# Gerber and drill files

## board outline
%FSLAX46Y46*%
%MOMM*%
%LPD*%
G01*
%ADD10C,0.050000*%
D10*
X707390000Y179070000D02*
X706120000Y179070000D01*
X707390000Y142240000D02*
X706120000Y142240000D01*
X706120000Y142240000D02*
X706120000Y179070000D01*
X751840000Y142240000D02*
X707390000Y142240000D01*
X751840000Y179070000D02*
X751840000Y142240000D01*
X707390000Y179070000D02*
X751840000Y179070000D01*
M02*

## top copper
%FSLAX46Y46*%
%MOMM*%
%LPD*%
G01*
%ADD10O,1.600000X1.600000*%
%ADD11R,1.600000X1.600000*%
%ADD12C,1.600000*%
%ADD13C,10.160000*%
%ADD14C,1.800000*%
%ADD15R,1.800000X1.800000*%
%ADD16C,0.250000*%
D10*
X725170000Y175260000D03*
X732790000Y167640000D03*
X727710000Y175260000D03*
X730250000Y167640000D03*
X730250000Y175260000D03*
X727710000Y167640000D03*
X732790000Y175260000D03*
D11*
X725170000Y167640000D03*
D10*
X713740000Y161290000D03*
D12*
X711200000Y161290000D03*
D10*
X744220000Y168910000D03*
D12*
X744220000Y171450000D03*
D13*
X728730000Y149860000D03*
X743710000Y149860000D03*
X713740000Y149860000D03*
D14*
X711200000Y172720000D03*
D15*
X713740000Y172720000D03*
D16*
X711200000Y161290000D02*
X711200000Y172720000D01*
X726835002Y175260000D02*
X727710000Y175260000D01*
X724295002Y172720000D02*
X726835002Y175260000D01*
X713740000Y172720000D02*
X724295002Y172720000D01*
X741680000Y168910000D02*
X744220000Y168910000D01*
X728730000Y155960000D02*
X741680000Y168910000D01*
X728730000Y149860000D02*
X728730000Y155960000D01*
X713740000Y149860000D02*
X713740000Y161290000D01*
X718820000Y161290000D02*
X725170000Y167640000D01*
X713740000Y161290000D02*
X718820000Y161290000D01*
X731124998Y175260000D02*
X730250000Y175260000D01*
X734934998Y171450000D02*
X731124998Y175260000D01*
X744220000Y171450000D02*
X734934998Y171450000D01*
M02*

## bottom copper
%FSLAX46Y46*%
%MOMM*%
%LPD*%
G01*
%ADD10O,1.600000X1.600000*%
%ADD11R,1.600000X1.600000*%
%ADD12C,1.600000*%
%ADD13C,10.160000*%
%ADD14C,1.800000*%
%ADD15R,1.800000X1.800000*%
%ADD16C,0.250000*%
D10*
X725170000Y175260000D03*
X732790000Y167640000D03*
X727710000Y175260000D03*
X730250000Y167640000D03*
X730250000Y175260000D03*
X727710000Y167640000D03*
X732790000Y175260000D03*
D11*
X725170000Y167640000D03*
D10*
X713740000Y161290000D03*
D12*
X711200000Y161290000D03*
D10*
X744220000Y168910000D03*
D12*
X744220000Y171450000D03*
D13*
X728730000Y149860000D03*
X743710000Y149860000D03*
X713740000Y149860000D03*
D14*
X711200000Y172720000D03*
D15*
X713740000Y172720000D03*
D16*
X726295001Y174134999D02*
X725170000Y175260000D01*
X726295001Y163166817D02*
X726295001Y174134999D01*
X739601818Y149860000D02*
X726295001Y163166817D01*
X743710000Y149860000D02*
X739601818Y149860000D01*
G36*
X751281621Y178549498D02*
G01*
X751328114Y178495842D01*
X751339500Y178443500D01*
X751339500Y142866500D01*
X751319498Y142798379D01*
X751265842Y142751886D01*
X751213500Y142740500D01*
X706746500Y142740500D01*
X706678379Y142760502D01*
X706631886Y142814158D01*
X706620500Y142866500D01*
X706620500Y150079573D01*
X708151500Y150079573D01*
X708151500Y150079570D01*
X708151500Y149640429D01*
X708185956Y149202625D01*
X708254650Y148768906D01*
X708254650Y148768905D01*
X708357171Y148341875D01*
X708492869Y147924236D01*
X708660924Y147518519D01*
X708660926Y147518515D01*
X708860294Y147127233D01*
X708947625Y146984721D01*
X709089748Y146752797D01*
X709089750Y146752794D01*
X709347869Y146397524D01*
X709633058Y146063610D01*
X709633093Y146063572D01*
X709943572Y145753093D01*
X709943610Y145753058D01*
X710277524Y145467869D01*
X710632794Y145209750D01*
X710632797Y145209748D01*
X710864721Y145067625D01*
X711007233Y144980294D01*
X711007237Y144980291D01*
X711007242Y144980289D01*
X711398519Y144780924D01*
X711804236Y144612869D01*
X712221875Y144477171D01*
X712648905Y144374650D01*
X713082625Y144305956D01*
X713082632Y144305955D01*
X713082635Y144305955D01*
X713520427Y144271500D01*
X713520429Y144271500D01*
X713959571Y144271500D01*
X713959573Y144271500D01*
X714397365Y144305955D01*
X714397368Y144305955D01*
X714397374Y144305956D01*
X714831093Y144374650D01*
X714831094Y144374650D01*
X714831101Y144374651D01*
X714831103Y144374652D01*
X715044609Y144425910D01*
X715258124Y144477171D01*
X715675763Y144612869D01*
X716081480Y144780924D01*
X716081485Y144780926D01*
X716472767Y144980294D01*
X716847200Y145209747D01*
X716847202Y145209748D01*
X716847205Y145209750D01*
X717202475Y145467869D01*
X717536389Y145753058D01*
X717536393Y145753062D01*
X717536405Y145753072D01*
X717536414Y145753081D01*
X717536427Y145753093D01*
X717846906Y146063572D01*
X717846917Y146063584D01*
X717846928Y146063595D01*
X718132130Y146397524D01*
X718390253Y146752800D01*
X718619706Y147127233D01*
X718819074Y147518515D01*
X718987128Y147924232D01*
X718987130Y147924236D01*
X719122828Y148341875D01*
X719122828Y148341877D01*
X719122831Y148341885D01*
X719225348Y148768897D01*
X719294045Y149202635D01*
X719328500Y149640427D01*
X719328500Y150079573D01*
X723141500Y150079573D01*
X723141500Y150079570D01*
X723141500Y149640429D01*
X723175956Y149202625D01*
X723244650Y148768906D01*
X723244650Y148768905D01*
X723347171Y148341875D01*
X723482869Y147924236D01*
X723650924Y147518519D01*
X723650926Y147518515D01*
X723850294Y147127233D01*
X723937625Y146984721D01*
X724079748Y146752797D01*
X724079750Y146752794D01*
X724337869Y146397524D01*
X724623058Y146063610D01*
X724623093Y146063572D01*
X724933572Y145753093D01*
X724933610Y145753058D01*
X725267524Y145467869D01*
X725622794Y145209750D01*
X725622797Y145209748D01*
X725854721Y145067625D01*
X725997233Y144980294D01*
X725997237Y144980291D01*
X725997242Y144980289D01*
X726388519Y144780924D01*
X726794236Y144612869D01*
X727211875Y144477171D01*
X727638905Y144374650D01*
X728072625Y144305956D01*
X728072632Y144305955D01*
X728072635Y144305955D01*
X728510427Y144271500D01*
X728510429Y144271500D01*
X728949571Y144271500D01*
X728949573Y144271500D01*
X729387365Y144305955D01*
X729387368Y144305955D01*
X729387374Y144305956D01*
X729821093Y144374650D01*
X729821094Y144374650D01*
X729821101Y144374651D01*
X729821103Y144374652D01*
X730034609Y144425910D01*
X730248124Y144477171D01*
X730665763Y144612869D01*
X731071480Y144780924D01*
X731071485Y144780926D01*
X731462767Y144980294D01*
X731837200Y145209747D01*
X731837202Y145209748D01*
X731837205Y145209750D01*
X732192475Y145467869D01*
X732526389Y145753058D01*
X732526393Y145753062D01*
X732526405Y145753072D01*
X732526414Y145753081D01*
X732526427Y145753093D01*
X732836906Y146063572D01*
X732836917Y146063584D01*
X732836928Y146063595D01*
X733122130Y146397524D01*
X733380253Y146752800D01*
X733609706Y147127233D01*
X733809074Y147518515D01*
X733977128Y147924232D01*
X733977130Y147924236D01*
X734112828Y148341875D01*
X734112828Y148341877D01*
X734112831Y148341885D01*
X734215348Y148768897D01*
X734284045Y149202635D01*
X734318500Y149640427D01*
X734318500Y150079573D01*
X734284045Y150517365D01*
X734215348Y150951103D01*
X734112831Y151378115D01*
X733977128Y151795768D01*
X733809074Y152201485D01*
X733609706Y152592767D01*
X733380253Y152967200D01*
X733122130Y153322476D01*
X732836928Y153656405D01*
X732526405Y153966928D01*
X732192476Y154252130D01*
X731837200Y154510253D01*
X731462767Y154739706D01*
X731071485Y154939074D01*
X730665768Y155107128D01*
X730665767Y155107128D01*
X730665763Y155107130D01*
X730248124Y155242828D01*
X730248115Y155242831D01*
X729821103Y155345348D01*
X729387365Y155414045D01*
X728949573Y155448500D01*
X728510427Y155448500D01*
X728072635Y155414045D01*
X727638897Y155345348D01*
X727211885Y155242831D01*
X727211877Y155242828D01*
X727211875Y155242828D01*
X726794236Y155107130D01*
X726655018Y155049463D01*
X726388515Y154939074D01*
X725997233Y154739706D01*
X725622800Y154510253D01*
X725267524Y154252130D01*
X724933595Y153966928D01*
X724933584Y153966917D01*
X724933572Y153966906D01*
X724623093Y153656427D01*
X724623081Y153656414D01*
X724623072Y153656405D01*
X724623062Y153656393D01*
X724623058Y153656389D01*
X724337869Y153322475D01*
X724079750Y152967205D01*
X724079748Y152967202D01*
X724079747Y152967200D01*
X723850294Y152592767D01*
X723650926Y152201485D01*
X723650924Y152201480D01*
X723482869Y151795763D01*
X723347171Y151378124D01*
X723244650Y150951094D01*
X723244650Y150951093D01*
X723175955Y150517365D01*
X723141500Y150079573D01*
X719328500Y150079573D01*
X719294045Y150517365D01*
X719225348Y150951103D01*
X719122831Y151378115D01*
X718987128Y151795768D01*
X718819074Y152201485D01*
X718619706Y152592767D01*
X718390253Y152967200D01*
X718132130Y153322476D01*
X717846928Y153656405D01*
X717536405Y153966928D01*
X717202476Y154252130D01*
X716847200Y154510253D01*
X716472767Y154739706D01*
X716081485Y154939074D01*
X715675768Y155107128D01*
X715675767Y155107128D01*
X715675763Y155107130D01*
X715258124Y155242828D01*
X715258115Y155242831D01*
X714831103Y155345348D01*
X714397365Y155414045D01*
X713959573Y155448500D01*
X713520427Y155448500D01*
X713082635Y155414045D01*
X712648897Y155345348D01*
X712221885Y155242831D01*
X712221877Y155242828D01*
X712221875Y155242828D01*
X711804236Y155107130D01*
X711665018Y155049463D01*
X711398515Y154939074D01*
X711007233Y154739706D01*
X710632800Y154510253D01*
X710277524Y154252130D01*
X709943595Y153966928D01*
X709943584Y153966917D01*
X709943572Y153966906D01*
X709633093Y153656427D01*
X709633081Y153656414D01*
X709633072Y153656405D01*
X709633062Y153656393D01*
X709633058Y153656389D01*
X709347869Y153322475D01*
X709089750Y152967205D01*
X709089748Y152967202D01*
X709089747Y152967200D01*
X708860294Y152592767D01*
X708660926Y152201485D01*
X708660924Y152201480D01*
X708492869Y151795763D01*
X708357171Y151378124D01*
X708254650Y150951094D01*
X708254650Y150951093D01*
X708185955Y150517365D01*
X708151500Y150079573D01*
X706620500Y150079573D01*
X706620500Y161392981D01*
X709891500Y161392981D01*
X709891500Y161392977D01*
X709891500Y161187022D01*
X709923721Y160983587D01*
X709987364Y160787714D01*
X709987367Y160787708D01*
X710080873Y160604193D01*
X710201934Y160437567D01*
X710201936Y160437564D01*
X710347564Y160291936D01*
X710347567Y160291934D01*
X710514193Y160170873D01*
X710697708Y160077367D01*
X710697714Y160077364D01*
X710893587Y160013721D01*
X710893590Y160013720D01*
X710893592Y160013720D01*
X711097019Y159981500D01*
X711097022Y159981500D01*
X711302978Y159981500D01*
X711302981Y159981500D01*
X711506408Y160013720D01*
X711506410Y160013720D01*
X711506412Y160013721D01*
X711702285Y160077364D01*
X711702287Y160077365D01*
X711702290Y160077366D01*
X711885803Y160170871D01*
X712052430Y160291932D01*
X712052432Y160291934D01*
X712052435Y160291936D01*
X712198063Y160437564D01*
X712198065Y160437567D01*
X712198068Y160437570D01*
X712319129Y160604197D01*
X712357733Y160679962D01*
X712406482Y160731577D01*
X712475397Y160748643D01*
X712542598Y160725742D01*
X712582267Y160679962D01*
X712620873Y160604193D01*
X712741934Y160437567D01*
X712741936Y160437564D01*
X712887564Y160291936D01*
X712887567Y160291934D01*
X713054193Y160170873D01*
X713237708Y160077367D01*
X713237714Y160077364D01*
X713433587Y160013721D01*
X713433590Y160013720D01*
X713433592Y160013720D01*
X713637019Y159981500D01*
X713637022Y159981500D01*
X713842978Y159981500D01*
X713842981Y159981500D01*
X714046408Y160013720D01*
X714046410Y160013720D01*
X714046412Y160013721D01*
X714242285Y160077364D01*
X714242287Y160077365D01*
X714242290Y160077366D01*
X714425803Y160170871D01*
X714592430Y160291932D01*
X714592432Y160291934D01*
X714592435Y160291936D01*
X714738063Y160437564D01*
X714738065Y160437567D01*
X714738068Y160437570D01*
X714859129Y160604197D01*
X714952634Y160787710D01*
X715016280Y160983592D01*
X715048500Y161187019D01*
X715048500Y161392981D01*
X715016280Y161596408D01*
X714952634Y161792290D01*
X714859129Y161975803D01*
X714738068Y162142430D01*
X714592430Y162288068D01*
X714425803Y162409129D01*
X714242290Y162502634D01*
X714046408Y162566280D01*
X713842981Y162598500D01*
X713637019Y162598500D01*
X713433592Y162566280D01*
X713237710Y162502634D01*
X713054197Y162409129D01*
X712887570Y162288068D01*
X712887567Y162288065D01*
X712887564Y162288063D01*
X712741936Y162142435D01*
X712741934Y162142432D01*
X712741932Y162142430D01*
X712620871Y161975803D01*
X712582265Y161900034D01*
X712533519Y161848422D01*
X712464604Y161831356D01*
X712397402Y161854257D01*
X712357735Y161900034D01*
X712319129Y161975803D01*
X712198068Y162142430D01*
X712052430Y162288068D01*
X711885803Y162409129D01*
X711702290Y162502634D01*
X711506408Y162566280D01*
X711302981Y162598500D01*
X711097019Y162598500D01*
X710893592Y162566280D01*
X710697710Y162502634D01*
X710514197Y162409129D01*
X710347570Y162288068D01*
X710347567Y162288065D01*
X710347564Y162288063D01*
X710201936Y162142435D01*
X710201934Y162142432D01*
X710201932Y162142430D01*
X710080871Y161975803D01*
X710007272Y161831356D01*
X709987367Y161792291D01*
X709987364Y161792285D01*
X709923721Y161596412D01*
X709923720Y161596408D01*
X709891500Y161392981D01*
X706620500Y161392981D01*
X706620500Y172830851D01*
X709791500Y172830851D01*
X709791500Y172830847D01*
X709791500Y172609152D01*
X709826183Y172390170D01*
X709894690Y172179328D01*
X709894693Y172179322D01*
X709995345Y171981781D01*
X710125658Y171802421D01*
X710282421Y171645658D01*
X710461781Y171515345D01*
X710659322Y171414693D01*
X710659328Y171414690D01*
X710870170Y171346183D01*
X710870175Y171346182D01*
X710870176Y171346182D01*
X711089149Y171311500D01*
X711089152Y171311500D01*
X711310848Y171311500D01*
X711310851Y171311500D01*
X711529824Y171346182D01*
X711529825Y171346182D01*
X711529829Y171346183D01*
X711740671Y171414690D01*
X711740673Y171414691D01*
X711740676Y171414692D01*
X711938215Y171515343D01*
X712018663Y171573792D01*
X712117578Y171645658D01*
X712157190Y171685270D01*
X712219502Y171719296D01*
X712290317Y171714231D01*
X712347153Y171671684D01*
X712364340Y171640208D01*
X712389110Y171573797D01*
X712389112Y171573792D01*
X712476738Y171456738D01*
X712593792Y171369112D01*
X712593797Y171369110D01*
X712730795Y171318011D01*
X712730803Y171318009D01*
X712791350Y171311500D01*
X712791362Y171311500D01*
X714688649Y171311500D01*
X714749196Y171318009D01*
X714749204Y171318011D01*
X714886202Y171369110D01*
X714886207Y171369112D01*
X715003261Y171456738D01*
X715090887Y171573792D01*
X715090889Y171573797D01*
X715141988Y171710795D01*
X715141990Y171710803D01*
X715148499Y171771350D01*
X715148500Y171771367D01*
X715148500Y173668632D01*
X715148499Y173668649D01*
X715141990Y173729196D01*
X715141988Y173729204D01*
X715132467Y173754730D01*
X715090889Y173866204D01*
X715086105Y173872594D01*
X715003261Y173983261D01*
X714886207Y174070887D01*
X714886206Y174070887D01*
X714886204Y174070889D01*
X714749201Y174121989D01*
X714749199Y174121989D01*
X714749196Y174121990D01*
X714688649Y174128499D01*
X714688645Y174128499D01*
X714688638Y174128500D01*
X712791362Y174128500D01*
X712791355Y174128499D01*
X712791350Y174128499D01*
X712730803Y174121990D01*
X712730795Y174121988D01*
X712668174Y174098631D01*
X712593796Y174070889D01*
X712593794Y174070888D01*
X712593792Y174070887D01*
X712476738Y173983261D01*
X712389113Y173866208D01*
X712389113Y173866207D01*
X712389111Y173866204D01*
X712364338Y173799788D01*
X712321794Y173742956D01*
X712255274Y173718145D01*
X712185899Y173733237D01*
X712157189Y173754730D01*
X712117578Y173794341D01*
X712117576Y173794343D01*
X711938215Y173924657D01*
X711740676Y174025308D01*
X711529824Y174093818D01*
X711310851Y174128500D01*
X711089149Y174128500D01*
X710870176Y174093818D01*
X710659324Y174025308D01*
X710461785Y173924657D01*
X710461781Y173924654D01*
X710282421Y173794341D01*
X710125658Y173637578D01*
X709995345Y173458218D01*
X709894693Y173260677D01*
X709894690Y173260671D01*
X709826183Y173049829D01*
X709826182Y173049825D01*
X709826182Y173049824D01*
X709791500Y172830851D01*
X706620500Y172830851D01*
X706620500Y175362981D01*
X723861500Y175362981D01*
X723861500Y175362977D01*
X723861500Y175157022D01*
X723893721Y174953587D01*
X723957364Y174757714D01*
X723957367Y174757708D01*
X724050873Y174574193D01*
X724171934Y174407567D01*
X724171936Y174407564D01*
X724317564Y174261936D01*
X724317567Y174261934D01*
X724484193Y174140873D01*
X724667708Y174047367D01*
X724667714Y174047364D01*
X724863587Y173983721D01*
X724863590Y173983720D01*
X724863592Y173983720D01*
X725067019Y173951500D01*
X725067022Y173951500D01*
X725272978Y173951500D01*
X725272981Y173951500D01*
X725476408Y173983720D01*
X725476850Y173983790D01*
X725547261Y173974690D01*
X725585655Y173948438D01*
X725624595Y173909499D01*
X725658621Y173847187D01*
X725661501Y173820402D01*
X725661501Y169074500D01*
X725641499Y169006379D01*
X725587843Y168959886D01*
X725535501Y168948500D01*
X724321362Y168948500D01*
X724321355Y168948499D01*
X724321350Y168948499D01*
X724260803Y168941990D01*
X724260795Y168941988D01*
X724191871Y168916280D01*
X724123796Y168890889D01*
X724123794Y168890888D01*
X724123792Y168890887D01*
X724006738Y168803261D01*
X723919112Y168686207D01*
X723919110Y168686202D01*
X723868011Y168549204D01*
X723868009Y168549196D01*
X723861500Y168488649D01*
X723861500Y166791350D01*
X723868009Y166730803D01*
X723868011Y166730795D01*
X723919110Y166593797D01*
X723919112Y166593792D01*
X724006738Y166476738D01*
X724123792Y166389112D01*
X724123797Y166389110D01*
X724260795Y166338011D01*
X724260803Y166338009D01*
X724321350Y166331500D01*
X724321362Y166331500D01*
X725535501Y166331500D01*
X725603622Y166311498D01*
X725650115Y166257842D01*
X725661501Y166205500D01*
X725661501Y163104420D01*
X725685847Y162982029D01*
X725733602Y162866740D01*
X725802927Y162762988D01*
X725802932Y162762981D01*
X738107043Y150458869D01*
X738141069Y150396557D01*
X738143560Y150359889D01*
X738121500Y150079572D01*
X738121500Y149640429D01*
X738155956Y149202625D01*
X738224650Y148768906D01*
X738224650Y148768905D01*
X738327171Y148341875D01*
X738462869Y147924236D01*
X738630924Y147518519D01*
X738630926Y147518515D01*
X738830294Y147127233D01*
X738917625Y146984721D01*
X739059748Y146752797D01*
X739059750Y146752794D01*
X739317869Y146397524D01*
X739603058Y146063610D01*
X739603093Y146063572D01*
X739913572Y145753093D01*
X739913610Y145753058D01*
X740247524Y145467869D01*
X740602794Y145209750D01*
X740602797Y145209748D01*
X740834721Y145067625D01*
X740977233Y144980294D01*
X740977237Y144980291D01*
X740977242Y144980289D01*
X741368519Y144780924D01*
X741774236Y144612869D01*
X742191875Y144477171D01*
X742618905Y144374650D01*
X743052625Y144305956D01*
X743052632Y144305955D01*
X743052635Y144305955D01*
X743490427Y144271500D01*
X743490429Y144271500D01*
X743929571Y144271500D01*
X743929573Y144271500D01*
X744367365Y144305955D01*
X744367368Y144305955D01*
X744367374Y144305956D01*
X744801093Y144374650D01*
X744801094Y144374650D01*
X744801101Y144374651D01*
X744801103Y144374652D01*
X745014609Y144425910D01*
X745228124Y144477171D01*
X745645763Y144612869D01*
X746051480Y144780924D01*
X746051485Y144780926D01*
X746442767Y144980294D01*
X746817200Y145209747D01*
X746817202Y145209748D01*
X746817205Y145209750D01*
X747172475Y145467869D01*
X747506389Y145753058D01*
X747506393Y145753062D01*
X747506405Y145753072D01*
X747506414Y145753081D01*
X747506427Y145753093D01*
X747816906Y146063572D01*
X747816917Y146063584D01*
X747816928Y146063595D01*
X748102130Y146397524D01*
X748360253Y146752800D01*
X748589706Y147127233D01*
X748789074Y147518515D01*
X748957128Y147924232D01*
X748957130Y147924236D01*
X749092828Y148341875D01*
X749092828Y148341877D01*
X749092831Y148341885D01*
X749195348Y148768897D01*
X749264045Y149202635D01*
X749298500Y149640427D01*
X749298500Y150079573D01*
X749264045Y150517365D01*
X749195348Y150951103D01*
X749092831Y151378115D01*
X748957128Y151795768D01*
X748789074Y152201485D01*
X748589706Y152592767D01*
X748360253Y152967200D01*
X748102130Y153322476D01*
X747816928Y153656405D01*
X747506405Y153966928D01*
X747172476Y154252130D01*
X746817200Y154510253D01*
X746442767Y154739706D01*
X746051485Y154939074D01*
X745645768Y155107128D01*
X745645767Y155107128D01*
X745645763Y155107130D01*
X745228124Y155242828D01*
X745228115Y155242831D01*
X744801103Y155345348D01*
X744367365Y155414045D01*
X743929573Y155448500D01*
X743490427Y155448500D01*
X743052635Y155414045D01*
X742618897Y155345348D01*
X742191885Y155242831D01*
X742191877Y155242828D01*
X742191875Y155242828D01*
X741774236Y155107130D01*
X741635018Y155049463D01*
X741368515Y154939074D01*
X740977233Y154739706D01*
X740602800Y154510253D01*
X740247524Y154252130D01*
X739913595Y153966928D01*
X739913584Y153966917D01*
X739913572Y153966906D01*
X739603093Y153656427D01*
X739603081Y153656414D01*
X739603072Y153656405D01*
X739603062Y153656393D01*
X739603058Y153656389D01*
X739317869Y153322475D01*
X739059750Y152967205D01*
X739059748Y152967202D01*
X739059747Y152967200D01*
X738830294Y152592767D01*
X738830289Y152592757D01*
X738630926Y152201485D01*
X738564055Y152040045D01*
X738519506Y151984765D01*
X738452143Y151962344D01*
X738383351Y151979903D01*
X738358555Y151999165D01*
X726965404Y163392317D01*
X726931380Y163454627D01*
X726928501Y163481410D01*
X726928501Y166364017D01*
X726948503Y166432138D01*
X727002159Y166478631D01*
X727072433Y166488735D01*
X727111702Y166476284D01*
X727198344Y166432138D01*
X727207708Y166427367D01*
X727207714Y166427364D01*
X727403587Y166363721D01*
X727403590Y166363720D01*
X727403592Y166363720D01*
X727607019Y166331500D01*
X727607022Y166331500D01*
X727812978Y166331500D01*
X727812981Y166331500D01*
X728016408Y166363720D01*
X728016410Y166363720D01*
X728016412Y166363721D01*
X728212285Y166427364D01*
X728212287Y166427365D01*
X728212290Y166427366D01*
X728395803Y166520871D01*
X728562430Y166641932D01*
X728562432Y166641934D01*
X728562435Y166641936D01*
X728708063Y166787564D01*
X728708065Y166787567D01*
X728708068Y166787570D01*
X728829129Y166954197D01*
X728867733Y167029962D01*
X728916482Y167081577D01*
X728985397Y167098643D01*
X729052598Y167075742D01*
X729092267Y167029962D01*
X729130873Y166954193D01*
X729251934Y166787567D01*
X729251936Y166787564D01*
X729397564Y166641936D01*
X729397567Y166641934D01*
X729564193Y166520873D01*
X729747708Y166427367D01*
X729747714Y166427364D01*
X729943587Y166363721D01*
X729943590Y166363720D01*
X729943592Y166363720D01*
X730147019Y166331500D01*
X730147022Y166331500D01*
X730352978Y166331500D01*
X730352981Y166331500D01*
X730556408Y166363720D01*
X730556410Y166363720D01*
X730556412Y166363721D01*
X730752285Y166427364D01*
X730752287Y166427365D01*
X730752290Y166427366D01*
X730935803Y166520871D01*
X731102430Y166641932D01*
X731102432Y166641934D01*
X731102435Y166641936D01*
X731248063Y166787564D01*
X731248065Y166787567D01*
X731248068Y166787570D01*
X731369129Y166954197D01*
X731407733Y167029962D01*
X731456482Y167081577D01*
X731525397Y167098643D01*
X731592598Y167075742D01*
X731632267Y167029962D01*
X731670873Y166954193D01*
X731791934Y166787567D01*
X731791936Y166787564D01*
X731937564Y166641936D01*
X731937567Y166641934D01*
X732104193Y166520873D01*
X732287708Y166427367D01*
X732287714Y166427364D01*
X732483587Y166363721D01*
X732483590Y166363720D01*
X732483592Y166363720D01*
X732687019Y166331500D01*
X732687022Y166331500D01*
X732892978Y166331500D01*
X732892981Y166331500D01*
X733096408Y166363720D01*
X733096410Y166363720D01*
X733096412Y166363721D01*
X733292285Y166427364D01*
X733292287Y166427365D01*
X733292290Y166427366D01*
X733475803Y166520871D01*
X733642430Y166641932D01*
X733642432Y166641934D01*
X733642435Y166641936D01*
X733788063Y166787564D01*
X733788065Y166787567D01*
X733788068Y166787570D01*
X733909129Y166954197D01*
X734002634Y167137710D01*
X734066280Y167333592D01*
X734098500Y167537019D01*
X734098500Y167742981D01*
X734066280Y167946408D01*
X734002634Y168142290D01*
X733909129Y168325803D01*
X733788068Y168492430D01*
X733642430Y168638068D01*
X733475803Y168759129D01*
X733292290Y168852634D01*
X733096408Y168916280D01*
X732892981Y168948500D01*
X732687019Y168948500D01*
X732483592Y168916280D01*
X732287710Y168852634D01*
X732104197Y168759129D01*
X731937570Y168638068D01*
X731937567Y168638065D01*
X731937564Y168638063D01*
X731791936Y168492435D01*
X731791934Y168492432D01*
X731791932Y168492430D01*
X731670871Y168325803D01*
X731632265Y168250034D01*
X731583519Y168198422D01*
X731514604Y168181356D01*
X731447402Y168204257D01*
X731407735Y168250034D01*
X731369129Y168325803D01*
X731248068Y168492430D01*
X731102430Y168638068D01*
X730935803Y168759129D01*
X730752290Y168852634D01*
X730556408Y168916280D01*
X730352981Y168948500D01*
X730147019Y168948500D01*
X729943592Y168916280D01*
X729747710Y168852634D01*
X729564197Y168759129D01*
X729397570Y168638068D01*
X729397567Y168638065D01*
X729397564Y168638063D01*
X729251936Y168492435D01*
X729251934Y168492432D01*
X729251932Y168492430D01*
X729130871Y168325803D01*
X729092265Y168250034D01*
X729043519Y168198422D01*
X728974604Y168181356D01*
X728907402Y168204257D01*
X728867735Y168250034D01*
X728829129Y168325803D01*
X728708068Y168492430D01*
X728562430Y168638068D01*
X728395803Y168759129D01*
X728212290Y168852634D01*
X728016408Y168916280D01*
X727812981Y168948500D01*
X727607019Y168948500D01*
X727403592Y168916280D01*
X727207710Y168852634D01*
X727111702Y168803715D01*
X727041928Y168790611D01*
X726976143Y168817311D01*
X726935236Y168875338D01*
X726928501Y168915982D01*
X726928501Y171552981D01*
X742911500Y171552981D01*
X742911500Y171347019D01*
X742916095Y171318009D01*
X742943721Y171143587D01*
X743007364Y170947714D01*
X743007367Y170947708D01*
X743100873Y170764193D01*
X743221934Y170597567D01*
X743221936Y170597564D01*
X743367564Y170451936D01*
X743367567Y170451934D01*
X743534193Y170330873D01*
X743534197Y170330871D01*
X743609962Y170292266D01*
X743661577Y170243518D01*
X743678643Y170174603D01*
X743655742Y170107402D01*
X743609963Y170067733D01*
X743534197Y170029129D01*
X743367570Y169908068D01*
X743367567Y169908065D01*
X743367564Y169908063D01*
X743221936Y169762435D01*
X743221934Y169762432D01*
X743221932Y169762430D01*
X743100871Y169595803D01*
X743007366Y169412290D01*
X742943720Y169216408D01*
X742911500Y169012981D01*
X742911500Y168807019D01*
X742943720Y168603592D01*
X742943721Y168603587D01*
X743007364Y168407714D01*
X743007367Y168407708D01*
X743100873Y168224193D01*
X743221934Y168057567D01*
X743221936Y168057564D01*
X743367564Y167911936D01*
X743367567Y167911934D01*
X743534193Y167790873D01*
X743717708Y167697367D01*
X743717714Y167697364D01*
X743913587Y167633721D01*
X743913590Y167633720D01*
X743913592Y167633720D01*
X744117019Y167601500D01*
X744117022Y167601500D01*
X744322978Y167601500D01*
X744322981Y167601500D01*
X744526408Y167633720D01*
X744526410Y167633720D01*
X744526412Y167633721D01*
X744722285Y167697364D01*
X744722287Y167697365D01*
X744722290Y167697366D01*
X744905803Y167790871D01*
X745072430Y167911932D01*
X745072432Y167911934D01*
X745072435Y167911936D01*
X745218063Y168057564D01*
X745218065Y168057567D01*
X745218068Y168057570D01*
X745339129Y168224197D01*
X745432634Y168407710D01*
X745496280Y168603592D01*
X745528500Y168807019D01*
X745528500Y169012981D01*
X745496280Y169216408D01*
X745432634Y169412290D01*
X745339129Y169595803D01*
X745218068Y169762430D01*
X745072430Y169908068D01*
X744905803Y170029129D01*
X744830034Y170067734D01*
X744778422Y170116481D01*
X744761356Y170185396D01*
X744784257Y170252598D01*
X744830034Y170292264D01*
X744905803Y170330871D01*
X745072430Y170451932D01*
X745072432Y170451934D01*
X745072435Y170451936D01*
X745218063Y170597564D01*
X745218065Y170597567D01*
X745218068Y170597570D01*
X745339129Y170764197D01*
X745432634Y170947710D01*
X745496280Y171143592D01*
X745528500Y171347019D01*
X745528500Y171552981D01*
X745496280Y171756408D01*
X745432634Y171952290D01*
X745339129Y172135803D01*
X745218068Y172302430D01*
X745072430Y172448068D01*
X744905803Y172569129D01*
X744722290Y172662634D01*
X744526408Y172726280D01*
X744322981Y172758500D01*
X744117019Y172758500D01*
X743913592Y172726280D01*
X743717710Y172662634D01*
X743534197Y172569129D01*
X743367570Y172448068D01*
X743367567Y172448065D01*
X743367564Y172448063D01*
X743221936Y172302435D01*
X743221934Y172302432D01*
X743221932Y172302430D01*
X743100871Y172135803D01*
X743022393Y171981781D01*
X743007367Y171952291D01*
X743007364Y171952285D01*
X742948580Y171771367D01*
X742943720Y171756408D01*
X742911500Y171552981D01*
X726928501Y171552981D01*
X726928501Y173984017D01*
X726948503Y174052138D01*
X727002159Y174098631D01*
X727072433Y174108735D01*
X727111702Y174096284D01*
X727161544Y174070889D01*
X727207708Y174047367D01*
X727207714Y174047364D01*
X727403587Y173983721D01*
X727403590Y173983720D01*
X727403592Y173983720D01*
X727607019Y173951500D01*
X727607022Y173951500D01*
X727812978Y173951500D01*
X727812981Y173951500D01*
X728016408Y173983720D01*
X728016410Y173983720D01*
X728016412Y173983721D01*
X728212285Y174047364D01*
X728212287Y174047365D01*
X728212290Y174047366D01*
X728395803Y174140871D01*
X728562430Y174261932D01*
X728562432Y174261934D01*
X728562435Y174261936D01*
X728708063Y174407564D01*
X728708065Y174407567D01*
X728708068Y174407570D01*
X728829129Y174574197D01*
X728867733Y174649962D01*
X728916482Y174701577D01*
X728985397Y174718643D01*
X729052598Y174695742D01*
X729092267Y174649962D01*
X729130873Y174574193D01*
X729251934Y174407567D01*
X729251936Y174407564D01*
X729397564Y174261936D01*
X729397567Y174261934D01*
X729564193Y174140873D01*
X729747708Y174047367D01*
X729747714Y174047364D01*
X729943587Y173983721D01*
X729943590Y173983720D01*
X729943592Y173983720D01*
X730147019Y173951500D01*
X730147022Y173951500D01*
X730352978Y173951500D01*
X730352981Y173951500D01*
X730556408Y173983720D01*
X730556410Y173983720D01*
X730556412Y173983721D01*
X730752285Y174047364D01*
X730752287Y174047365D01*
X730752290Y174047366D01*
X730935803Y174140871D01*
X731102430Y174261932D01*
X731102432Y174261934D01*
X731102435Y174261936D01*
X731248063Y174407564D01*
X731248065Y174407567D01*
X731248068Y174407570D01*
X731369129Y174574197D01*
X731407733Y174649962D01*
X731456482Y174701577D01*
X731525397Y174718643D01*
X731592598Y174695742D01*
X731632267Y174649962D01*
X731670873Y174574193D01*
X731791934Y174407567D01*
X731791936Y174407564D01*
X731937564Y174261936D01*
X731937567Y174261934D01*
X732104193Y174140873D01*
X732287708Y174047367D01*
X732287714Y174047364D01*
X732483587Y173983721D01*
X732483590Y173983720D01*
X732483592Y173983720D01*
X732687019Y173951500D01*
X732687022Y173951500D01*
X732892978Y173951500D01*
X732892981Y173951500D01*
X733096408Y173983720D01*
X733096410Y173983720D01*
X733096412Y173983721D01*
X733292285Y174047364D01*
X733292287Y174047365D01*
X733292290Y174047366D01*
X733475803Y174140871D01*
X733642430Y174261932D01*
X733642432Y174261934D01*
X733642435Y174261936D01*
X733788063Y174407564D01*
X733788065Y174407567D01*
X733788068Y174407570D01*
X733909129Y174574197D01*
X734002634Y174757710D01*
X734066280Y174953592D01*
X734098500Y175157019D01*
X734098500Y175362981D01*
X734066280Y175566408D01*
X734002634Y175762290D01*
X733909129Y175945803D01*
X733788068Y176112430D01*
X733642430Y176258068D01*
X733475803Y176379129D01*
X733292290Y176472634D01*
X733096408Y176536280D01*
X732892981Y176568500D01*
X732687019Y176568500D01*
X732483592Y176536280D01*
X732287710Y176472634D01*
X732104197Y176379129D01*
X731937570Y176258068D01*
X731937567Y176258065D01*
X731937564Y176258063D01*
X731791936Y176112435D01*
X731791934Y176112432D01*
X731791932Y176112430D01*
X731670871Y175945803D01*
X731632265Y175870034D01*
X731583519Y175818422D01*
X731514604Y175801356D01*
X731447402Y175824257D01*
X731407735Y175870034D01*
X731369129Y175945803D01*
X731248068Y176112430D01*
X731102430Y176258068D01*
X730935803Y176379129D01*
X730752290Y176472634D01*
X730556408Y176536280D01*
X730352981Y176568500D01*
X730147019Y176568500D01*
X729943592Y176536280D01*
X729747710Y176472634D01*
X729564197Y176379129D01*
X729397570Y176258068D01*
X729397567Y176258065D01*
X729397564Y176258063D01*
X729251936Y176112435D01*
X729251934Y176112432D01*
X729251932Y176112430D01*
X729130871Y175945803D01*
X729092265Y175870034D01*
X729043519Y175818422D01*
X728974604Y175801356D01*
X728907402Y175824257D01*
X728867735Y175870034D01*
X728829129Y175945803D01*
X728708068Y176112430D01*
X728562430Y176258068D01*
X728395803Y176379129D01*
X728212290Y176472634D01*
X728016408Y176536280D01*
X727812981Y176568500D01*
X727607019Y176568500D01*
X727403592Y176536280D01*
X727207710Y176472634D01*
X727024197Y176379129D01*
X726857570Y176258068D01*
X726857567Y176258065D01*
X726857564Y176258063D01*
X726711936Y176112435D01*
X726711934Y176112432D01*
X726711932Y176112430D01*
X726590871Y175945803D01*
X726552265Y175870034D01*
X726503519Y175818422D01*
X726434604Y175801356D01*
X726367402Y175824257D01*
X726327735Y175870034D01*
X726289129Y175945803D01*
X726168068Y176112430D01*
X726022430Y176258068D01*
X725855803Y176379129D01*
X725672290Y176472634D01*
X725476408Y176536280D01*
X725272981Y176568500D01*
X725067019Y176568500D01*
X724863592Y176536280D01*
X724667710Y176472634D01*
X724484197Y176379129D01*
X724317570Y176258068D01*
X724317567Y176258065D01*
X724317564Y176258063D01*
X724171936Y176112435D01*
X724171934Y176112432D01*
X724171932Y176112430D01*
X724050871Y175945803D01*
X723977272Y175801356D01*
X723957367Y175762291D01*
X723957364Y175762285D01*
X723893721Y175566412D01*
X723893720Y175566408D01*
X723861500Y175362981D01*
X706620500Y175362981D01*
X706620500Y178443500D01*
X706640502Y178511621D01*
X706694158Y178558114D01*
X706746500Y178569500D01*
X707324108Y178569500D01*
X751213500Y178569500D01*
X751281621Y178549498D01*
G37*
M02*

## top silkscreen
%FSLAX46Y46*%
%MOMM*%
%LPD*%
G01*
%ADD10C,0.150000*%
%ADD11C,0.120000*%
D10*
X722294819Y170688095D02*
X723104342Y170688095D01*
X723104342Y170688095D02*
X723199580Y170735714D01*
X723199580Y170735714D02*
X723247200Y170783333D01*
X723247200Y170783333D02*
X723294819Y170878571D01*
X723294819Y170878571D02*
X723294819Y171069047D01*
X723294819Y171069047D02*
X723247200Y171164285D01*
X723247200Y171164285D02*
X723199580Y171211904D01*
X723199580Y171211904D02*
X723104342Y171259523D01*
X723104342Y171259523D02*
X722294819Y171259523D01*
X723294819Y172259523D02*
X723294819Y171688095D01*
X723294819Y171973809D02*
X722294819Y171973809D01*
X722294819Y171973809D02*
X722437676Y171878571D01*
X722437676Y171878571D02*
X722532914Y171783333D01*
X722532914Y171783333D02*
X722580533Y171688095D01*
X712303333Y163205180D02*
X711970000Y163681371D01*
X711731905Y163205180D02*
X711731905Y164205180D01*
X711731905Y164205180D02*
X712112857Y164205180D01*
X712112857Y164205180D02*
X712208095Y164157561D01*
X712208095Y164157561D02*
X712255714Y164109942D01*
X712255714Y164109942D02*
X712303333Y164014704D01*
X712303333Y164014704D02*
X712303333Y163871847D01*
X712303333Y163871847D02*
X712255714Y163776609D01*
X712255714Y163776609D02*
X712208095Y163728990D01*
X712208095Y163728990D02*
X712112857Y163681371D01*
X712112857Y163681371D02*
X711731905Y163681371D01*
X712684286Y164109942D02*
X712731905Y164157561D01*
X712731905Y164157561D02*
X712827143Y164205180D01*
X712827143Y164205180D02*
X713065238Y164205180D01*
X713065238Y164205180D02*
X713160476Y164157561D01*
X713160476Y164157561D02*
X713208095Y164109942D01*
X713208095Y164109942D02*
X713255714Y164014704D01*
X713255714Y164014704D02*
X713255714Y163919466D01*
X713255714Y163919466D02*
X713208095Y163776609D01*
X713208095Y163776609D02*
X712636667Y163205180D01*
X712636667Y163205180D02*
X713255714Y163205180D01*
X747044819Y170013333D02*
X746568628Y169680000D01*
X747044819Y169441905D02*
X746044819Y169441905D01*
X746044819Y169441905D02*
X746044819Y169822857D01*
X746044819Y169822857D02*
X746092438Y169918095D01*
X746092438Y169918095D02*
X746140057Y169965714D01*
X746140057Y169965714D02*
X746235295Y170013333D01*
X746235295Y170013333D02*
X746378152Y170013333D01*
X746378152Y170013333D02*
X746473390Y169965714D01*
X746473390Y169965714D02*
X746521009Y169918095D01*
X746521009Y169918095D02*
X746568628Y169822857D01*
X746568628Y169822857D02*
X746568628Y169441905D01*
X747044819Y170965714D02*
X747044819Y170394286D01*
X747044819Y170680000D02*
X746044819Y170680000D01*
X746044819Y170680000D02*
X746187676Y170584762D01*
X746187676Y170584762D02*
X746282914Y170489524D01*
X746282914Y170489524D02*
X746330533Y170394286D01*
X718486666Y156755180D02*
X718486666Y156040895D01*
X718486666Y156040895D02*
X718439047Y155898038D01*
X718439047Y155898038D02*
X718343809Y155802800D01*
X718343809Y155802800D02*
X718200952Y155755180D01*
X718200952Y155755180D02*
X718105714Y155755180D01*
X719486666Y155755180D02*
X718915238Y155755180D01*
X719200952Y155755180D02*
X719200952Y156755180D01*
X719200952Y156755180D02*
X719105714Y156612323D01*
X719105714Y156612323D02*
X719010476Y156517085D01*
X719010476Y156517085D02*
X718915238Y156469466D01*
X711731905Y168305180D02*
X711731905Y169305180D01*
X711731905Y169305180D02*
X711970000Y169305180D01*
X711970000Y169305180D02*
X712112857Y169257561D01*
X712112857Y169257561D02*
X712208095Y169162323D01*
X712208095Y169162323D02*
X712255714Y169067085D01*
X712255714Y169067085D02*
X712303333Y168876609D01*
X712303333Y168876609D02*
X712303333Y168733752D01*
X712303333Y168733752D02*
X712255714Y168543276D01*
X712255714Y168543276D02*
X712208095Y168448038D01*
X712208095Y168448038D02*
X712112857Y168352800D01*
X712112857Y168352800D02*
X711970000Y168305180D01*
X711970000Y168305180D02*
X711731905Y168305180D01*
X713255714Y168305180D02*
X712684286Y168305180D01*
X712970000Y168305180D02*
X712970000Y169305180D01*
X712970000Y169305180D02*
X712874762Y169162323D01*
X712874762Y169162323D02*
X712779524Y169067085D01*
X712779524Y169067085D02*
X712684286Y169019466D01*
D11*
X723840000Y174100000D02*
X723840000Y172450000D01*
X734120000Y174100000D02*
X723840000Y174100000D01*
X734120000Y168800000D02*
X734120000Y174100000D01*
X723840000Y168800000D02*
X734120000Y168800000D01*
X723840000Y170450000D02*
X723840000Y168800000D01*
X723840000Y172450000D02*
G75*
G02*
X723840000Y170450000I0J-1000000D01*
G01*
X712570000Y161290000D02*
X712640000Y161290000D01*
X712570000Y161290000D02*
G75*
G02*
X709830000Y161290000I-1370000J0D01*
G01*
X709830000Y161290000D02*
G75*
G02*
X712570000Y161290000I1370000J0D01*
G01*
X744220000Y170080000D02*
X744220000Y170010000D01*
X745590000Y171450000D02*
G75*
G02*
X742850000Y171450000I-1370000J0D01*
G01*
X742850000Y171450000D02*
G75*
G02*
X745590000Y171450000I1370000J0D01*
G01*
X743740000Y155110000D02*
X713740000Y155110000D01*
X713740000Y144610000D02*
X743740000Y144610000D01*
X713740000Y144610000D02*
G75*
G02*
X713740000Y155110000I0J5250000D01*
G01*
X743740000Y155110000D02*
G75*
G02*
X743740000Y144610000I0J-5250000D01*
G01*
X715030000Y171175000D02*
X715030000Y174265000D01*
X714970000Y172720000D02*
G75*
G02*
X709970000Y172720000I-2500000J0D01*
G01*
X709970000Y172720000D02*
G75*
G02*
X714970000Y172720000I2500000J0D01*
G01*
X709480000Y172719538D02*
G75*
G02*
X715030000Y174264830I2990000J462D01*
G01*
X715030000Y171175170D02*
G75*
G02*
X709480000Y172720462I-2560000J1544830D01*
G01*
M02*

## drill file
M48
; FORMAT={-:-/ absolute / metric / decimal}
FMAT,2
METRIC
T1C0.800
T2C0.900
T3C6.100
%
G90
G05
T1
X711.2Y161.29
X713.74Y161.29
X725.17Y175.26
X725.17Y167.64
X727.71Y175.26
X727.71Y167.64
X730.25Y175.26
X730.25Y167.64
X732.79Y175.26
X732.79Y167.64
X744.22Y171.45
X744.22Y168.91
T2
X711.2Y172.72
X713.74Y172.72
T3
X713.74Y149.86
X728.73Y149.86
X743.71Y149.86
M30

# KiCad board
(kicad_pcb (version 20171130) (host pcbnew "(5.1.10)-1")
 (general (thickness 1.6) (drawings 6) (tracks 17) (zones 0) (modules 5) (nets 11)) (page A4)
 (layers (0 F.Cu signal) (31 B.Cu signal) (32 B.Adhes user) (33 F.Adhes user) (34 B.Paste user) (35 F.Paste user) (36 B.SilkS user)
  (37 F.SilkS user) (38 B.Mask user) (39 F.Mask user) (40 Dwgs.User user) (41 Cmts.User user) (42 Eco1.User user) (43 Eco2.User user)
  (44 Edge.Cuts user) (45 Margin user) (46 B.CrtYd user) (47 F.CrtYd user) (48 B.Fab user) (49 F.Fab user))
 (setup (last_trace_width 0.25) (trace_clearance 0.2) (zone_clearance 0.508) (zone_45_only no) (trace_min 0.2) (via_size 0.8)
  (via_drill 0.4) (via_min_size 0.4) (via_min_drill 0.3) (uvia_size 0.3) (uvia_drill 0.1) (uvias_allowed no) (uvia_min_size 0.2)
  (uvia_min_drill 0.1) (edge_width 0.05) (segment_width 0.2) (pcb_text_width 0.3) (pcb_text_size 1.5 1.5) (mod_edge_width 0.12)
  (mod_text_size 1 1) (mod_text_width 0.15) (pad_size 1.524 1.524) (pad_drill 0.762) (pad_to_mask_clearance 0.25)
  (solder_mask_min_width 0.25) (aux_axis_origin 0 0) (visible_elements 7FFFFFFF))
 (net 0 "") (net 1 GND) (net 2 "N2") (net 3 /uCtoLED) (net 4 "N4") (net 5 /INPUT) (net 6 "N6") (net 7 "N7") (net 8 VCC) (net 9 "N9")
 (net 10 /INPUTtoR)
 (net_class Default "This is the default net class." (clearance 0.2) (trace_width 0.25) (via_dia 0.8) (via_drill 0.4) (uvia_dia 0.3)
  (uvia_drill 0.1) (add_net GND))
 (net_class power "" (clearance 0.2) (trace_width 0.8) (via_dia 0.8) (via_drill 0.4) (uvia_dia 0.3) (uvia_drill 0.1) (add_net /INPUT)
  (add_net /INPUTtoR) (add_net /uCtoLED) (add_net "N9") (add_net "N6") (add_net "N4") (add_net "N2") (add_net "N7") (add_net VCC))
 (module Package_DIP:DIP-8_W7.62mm (layer F.Cu) (at 725.17 -167.64 90)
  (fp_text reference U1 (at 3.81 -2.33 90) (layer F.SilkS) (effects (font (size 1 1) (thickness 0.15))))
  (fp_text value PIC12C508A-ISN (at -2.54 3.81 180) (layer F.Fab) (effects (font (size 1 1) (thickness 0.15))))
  (fp_line (start 6.46 -1.33) (end 4.81 -1.33) (layer F.SilkS) (width 0.12))
  (fp_line (start 6.46 8.95) (end 6.46 -1.33) (layer F.SilkS) (width 0.12))
  (fp_line (start 1.16 8.95) (end 6.46 8.95) (layer F.SilkS) (width 0.12))
  (fp_line (start 1.16 -1.33) (end 1.16 8.95) (layer F.SilkS) (width 0.12))
  (fp_line (start 2.81 -1.33) (end 1.16 -1.33) (layer F.SilkS) (width 0.12))
  (fp_arc (start 3.81 -1.33) (end 2.81 -1.33) (angle -180) (layer F.SilkS) (width 0.12))
  (pad 8 thru_hole oval (at 7.62 0 90) (size 1.6 1.6) (drill 0.8) (layers *.Cu *.Mask) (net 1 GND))
  (pad 4 thru_hole oval (at 0 7.62 90) (size 1.6 1.6) (drill 0.8) (layers *.Cu *.Mask) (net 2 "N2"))
  (pad 7 thru_hole oval (at 7.62 2.54 90) (size 1.6 1.6) (drill 0.8) (layers *.Cu *.Mask) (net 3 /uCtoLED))
  (pad 3 thru_hole oval (at 0 5.08 90) (size 1.6 1.6) (drill 0.8) (layers *.Cu *.Mask) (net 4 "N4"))
  (pad 6 thru_hole oval (at 7.62 5.08 90) (size 1.6 1.6) (drill 0.8) (layers *.Cu *.Mask) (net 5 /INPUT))
  (pad 2 thru_hole oval (at 0 2.54 90) (size 1.6 1.6) (drill 0.8) (layers *.Cu *.Mask) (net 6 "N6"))
  (pad 5 thru_hole oval (at 7.62 7.62 90) (size 1.6 1.6) (drill 0.8) (layers *.Cu *.Mask) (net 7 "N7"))
  (pad 1 thru_hole rect (at 0 0 90) (size 1.6 1.6) (drill 0.8) (layers *.Cu *.Mask) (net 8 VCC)))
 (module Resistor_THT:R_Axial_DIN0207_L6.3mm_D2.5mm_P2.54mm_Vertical (layer F.Cu) (at 711.2 -161.29)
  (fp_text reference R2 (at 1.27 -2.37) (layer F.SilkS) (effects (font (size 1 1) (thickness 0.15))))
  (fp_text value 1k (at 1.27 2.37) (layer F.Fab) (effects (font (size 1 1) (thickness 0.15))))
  (fp_line (start 1.37 0) (end 1.44 0) (layer F.SilkS) (width 0.12))
  (fp_circle (center 0 0) (end 1.37 0) (layer F.SilkS) (width 0.12))
  (pad 2 thru_hole oval (at 2.54 0) (size 1.6 1.6) (drill 0.8) (layers *.Cu *.Mask) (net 8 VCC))
  (pad 1 thru_hole circle (at 0 0) (size 1.6 1.6) (drill 0.8) (layers *.Cu *.Mask) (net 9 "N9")))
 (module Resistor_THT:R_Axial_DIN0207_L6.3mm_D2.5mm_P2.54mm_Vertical (layer F.Cu) (at 744.22 -171.45 270)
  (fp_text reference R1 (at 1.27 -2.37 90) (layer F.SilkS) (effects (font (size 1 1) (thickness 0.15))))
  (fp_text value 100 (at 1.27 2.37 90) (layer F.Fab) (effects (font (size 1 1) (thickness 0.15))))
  (fp_line (start 1.37 0) (end 1.44 0) (layer F.SilkS) (width 0.12))
  (fp_circle (center 0 0) (end 1.37 0) (layer F.SilkS) (width 0.12))
  (pad 2 thru_hole oval (at 2.54 0 270) (size 1.6 1.6) (drill 0.8) (layers *.Cu *.Mask) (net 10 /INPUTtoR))
  (pad 1 thru_hole circle (at 0 0 270) (size 1.6 1.6) (drill 0.8) (layers *.Cu *.Mask) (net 5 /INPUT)))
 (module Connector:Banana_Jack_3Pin (layer F.Cu) (at 713.74 -149.86)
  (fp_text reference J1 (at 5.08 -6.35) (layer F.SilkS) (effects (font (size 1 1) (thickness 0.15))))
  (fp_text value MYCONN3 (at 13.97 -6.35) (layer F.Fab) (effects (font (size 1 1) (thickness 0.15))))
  (fp_line (start 30 -5.25) (end 0 -5.25) (layer F.SilkS) (width 0.12))
  (fp_line (start 0 5.25) (end 30 5.25) (layer F.SilkS) (width 0.12))
  (fp_arc (start 0 0) (end 0 5.25) (angle 180) (layer F.SilkS) (width 0.12))
  (fp_arc (start 30 0) (end 30 -5.25) (angle 180) (layer F.SilkS) (width 0.12))
  (pad 2 thru_hole circle (at 14.99 0) (size 10.16 10.16) (drill 6.1) (layers *.Cu *.Mask) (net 10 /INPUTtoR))
  (pad 3 thru_hole circle (at 29.97 0) (size 10.16 10.16) (drill 6.1) (layers *.Cu *.Mask) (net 1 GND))
  (pad 1 thru_hole circle (at 0 0) (size 10.16 10.16) (drill 6.1) (layers *.Cu *.Mask) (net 8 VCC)))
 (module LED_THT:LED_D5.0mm (layer F.Cu) (at 713.74 -172.72 180)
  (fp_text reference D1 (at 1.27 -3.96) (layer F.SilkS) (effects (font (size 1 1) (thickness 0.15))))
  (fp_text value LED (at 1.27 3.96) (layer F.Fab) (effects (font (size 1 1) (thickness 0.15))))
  (fp_line (start -1.29 -1.545) (end -1.29 1.545) (layer F.SilkS) (width 0.12))
  (fp_circle (center 1.27 0) (end 3.77 0) (layer F.SilkS) (width 0.12))
  (fp_arc (start 1.27 0) (end -1.29 1.54483) (angle -148.9) (layer F.SilkS) (width 0.12))
  (fp_arc (start 1.27 0) (end -1.29 -1.54483) (angle 148.9) (layer F.SilkS) (width 0.12))
  (pad 2 thru_hole circle (at 2.54 0 180) (size 1.8 1.8) (drill 0.9) (layers *.Cu *.Mask) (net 9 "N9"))
  (pad 1 thru_hole rect (at 0 0 180) (size 1.8 1.8) (drill 0.9) (layers *.Cu *.Mask) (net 3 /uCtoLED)))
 (gr_line (start 707.39 -179.07) (end 706.12 -179.07) (layer Edge.Cuts) (width 0.05))
 (gr_line (start 707.39 -142.24) (end 706.12 -142.24) (layer Edge.Cuts) (width 0.05))
 (gr_line (start 706.12 -142.24) (end 706.12 -179.07) (layer Edge.Cuts) (width 0.05))
 (gr_line (start 751.84 -142.24) (end 707.39 -142.24) (layer Edge.Cuts) (width 0.05))
 (gr_line (start 751.84 -179.07) (end 751.84 -142.24) (layer Edge.Cuts) (width 0.05))
 (gr_line (start 707.39 -179.07) (end 751.84 -179.07) (layer Edge.Cuts) (width 0.05))
 (segment (start 711.2 -161.29) (end 711.2 -172.72) (width 0.25) (layer F.Cu) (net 9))
 (segment (start 726.835002 -175.26) (end 727.71 -175.26) (width 0.25) (layer F.Cu) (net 3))
 (segment (start 724.295002 -172.72) (end 726.835002 -175.26) (width 0.25) (layer F.Cu) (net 3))
 (segment (start 713.74 -172.72) (end 724.295002 -172.72) (width 0.25) (layer F.Cu) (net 3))
 (segment (start 741.68 -168.91) (end 744.22 -168.91) (width 0.25) (layer F.Cu) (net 10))
 (segment (start 728.73 -155.96) (end 741.68 -168.91) (width 0.25) (layer F.Cu) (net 10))
 (segment (start 728.73 -149.86) (end 728.73 -155.96) (width 0.25) (layer F.Cu) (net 10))
 (segment (start 726.295001 -174.134999) (end 725.17 -175.26) (width 0.25) (layer B.Cu) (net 1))
 (segment (start 726.295001 -163.166817) (end 726.295001 -174.134999) (width 0.25) (layer B.Cu) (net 1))
 (segment (start 739.601818 -149.86) (end 726.295001 -163.166817) (width 0.25) (layer B.Cu) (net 1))
 (segment (start 743.71 -149.86) (end 739.601818 -149.86) (width 0.25) (layer B.Cu) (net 1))
 (segment (start 713.74 -149.86) (end 713.74 -161.29) (width 0.25) (layer F.Cu) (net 8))
 (segment (start 718.82 -161.29) (end 725.17 -167.64) (width 0.25) (layer F.Cu) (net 8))
 (segment (start 713.74 -161.29) (end 718.82 -161.29) (width 0.25) (layer F.Cu) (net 8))
 (segment (start 731.124998 -175.26) (end 730.25 -175.26) (width 0.25) (layer F.Cu) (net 5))
 (segment (start 734.934998 -171.45) (end 731.124998 -175.26) (width 0.25) (layer F.Cu) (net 5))
 (segment (start 744.22 -171.45) (end 734.934998 -171.45) (width 0.25) (layer F.Cu) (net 5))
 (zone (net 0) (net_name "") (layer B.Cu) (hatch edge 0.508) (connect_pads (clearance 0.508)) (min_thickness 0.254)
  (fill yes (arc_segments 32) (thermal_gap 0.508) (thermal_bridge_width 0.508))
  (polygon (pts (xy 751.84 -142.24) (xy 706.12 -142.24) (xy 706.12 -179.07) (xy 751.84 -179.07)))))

